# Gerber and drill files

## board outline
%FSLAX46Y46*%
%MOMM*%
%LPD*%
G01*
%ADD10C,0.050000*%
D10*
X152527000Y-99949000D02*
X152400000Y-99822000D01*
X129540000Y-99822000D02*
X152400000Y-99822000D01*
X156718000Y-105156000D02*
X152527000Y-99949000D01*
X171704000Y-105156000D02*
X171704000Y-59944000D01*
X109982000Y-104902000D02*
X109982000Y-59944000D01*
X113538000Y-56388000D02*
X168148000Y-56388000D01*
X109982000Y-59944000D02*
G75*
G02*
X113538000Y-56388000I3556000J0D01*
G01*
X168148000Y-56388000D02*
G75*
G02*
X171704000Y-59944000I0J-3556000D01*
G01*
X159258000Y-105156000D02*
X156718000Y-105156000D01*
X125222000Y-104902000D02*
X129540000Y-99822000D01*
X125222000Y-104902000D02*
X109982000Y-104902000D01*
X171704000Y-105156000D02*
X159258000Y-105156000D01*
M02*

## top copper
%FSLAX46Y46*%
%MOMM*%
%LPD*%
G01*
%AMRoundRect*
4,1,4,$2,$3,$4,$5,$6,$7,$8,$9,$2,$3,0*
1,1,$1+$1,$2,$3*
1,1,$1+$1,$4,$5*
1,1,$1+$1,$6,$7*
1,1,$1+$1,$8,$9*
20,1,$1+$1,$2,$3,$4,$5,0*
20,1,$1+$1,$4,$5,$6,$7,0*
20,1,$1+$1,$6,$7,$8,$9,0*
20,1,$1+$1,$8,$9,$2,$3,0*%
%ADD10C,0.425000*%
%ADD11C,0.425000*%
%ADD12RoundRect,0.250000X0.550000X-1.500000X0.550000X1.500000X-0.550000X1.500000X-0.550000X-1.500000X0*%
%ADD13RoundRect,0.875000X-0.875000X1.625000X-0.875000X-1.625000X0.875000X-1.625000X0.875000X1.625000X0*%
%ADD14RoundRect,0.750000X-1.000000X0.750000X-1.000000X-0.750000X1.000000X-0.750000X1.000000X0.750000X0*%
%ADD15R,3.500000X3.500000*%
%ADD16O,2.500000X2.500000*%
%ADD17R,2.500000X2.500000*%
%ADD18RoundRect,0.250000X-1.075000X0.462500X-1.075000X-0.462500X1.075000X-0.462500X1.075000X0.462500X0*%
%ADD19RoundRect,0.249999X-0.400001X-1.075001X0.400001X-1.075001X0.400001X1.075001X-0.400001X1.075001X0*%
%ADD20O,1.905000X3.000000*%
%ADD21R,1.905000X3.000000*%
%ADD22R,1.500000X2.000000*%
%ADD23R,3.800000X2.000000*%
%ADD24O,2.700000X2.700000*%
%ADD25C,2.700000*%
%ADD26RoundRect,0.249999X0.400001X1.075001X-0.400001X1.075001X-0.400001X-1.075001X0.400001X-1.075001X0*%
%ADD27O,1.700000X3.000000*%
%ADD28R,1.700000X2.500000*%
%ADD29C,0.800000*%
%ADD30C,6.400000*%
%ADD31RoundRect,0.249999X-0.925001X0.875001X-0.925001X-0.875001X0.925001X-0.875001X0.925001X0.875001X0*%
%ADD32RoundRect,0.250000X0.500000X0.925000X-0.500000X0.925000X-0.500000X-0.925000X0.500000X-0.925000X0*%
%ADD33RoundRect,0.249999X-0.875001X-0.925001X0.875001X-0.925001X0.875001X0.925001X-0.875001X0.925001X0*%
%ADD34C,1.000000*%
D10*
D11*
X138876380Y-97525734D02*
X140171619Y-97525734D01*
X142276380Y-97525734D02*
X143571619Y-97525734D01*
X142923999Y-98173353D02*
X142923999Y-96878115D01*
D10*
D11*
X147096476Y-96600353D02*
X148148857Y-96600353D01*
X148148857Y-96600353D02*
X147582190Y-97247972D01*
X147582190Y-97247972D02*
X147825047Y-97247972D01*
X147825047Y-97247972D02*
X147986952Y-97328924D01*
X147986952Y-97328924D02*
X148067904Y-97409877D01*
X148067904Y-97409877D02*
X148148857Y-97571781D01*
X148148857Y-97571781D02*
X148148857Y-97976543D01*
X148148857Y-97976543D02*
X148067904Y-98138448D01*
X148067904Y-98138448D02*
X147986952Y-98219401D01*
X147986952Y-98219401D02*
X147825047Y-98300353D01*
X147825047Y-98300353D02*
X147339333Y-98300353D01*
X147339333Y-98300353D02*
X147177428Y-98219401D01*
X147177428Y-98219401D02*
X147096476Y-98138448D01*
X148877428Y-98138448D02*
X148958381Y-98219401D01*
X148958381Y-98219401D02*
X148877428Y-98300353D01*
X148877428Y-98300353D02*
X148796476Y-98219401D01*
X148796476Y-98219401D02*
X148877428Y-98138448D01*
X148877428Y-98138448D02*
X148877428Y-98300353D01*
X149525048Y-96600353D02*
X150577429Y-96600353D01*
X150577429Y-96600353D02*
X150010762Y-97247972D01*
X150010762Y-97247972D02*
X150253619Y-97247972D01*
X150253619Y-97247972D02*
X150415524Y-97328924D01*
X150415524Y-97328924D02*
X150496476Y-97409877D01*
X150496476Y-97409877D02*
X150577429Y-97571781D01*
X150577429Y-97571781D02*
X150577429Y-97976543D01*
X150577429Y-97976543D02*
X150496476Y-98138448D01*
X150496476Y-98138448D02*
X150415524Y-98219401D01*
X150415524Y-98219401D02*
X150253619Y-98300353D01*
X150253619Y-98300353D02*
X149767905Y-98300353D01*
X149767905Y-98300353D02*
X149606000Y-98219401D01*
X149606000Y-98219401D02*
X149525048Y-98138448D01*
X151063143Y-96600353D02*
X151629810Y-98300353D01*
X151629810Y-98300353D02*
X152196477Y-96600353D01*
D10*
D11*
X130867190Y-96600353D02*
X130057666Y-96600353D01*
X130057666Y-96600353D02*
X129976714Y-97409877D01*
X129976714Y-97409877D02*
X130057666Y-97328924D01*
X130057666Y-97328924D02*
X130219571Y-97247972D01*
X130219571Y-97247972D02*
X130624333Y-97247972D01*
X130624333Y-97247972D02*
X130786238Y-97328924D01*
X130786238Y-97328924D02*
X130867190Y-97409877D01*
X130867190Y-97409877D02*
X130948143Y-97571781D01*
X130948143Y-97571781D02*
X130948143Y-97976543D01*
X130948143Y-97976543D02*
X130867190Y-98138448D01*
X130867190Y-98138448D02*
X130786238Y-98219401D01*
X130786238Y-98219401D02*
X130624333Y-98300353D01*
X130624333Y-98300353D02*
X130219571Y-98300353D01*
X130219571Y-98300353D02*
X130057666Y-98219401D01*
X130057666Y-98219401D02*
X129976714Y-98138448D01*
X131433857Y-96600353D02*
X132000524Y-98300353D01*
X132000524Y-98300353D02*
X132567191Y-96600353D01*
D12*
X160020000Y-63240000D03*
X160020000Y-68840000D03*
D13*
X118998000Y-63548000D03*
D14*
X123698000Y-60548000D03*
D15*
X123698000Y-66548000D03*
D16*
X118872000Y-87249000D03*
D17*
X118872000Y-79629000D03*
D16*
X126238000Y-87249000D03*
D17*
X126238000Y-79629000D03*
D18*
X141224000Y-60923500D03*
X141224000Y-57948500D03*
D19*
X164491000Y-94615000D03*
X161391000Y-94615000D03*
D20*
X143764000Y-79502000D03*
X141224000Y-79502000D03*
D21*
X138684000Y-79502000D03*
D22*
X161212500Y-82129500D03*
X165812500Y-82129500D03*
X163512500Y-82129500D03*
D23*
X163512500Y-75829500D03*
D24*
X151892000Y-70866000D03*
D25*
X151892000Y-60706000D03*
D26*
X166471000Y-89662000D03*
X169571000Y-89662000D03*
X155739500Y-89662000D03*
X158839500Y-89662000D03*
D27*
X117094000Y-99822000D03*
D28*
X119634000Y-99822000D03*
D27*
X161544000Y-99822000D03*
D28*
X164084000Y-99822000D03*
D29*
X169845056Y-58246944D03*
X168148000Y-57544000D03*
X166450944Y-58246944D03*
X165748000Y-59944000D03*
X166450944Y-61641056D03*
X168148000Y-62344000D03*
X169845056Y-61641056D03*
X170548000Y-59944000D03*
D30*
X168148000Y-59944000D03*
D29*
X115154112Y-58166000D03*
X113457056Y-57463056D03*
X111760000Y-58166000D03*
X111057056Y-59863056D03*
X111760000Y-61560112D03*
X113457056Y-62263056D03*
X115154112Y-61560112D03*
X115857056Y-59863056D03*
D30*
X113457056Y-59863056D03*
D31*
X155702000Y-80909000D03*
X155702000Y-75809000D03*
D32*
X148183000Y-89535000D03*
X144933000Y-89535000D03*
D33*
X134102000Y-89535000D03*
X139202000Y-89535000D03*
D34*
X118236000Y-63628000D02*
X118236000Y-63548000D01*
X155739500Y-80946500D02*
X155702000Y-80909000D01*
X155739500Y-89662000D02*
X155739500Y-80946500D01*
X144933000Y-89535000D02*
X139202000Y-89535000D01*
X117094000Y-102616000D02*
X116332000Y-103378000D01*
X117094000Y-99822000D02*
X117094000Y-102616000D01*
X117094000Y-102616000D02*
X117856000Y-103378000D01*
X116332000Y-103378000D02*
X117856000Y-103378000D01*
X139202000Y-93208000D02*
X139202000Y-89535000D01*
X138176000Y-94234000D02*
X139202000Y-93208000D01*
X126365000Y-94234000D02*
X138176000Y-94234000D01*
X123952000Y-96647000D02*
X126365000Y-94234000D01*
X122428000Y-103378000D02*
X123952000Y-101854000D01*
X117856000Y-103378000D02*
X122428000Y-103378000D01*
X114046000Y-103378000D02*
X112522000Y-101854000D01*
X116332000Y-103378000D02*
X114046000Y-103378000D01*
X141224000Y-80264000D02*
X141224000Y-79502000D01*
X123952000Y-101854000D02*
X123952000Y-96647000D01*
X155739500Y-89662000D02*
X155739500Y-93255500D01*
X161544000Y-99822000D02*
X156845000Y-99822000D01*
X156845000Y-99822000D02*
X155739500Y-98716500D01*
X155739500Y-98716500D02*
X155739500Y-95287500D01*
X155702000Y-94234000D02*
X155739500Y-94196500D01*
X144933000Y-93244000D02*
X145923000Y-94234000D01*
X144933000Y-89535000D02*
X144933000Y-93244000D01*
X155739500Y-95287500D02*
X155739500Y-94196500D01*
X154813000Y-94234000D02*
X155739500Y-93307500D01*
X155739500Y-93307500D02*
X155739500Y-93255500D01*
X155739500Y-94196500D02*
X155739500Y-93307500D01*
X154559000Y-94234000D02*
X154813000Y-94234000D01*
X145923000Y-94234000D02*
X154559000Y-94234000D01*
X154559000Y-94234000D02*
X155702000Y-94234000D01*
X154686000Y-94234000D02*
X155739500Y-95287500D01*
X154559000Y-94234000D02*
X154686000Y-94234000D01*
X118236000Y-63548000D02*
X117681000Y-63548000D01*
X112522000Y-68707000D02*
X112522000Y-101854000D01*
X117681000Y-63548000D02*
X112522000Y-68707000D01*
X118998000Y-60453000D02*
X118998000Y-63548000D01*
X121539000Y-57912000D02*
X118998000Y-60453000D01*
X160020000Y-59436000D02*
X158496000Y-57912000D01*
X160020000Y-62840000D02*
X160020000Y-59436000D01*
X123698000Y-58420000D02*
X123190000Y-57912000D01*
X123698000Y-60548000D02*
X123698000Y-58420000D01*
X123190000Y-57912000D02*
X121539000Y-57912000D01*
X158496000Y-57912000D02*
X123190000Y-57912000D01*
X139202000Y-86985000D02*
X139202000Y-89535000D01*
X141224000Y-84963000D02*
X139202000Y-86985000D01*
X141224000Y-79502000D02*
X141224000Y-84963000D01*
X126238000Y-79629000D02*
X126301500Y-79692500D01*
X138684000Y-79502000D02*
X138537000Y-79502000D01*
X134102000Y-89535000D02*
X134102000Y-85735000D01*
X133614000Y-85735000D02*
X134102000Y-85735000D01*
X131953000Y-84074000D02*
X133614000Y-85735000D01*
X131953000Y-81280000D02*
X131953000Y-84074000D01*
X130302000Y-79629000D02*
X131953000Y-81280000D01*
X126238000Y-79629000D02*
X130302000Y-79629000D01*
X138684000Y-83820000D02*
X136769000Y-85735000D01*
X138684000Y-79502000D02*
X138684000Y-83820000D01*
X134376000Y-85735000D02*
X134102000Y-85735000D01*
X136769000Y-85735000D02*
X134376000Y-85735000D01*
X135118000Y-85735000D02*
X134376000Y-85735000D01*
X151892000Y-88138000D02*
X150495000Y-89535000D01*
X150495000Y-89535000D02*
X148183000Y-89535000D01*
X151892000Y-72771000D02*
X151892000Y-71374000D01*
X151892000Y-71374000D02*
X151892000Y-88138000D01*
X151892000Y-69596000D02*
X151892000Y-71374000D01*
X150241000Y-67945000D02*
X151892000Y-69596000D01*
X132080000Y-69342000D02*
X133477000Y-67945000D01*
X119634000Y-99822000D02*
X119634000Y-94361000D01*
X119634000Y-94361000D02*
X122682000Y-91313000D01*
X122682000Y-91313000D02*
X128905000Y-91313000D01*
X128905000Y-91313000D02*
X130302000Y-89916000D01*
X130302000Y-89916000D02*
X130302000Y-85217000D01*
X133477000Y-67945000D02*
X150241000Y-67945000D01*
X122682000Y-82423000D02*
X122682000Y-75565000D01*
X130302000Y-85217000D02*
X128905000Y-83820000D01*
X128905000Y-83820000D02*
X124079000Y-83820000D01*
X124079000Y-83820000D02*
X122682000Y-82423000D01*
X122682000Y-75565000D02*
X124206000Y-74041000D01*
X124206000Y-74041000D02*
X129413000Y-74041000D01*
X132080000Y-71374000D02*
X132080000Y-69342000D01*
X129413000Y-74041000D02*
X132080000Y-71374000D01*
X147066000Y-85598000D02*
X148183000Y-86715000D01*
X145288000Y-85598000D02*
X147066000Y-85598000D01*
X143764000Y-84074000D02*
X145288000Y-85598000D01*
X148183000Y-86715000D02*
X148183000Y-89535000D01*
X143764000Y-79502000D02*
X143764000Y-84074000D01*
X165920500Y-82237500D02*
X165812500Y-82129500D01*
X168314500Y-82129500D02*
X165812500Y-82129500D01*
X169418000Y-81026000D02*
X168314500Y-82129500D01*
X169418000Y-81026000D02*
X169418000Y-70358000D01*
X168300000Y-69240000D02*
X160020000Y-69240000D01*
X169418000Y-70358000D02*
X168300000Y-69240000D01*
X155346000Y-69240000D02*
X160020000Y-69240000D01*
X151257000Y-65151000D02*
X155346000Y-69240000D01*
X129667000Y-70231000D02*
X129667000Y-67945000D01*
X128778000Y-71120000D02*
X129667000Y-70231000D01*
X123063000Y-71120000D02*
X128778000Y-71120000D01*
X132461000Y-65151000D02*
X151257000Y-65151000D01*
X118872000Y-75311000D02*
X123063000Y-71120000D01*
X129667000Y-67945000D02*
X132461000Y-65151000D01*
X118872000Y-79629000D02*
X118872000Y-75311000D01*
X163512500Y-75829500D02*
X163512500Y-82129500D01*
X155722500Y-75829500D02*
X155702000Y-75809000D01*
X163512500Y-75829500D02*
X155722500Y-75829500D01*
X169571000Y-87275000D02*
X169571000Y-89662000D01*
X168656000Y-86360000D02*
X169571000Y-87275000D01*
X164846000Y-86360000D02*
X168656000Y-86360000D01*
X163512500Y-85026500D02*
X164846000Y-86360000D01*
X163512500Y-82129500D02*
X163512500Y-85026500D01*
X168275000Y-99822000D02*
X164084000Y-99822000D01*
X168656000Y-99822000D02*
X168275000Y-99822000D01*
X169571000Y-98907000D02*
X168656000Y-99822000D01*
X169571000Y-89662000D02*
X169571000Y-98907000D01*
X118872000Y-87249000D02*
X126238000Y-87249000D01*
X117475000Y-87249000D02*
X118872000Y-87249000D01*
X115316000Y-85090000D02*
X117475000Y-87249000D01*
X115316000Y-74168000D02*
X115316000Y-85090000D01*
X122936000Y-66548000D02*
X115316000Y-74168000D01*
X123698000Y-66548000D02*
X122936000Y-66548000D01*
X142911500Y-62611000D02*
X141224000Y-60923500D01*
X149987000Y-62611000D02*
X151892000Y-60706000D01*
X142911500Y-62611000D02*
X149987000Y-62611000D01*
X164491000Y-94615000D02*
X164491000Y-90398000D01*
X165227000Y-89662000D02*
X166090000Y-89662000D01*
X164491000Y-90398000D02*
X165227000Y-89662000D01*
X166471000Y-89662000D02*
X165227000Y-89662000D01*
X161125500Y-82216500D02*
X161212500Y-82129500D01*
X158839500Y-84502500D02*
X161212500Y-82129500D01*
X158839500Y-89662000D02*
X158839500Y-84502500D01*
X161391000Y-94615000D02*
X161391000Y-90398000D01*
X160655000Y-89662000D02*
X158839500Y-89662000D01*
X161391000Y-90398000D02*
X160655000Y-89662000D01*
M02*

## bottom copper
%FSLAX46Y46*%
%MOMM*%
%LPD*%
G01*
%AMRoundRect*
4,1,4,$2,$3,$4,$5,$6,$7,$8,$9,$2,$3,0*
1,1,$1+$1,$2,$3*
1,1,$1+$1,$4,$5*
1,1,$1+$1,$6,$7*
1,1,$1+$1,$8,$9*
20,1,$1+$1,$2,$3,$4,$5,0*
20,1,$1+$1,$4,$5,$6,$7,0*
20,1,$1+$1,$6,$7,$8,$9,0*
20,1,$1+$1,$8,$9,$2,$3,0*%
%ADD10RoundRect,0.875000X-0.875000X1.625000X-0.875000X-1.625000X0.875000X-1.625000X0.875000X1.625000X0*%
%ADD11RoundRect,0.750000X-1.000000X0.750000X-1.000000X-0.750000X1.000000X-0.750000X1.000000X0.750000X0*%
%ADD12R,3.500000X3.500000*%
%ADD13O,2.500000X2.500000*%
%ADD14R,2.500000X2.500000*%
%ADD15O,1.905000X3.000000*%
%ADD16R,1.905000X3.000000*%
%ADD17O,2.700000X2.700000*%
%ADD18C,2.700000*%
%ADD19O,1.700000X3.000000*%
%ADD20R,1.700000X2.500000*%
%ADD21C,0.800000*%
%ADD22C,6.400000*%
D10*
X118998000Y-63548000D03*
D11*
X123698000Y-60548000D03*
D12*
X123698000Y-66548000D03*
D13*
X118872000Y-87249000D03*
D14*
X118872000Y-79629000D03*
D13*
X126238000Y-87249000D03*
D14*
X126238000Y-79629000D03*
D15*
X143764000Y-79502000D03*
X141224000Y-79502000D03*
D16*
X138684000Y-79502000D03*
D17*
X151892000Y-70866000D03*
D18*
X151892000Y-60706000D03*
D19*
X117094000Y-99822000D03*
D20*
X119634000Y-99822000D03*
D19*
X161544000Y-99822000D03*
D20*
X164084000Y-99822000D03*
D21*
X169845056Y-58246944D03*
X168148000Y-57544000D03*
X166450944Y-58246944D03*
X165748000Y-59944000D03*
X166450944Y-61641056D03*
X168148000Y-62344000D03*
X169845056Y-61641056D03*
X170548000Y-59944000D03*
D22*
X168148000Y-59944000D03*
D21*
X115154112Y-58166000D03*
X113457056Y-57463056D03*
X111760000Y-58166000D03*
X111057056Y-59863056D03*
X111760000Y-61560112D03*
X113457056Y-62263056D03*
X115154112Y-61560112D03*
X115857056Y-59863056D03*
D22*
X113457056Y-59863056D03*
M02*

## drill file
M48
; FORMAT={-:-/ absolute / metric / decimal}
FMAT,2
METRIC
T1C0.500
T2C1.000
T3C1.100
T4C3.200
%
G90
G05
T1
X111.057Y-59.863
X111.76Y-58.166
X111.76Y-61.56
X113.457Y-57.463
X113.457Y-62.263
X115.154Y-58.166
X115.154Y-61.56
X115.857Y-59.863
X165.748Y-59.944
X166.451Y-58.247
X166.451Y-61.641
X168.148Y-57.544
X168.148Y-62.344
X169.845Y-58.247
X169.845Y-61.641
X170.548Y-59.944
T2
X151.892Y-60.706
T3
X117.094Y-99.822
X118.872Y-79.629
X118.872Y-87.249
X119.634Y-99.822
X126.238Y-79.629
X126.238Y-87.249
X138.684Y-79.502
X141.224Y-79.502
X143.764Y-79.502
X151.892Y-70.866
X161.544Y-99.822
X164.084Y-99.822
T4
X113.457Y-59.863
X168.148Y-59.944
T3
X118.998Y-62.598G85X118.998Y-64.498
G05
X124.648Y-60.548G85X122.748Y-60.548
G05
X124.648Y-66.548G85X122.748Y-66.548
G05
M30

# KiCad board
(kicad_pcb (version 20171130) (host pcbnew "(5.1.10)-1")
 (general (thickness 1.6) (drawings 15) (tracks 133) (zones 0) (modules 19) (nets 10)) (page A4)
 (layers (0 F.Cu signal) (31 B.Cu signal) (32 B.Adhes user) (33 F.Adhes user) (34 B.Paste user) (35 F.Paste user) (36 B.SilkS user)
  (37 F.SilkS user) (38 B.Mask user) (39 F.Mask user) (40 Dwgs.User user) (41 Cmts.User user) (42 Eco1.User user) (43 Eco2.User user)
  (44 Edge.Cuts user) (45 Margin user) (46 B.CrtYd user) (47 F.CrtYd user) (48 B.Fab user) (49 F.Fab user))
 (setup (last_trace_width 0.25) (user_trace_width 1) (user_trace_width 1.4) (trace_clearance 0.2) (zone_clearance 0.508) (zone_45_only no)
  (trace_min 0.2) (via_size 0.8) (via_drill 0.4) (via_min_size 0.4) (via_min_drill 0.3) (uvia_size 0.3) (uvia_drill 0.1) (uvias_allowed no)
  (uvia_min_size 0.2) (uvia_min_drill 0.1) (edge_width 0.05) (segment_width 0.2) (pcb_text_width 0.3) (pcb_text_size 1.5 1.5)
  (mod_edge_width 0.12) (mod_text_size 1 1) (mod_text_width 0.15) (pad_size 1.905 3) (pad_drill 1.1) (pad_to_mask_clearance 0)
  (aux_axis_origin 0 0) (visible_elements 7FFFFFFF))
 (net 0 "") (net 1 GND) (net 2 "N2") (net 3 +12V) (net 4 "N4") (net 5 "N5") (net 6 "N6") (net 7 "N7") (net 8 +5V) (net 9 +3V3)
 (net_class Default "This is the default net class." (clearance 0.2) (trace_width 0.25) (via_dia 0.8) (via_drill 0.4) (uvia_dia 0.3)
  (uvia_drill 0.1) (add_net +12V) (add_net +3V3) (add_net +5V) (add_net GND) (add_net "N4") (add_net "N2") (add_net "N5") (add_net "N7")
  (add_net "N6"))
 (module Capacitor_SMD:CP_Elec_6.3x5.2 (layer F.Cu) (at 160.02 66.04 90)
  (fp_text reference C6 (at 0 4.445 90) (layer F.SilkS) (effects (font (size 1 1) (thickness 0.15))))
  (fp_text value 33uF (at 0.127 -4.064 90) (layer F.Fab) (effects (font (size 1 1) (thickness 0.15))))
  (pad 2 smd roundrect (at 2.8 0 90) (size 3.5 1.6) (layers F.Cu F.Paste F.Mask) (roundrect_rratio 0.15625) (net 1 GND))
  (pad 1 smd roundrect (at -2.8 0 90) (size 3.5 1.6) (layers F.Cu F.Paste F.Mask) (roundrect_rratio 0.15625) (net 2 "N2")))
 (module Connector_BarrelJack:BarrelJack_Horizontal (layer F.Cu) (at 123.698 66.548 270)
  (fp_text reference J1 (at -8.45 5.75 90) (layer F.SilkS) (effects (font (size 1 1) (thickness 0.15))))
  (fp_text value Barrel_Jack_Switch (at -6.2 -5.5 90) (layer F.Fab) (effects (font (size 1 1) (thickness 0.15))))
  (pad 3 thru_hole roundrect (at -3 4.7 270) (size 5 3.5) (drill oval 3 1.1) (layers *.Cu *.Mask) (roundrect_rratio 0.25) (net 1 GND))
  (pad 2 thru_hole roundrect (at -6 0 270) (size 3 3.5) (drill oval 1.1 3) (layers *.Cu *.Mask) (roundrect_rratio 0.25) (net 1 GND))
  (pad 1 thru_hole rect (at 0 0 270) (size 3.5 3.5) (drill oval 1.1 3) (layers *.Cu *.Mask) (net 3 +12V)))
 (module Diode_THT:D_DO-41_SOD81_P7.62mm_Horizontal (layer F.Cu) (at 118.872 79.629 270)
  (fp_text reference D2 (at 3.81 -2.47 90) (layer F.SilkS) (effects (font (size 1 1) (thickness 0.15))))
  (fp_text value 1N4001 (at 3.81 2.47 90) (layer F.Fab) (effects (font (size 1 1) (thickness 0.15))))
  (pad 2 thru_hole oval (at 7.62 0 270) (size 2.5 2.5) (drill 1.1) (layers *.Cu *.Mask) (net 3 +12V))
  (pad 1 thru_hole rect (at 0 0 270) (size 2.5 2.5) (drill 1.1) (layers *.Cu *.Mask) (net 2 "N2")))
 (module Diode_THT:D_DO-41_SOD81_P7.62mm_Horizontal (layer F.Cu) (at 126.238 79.629 270)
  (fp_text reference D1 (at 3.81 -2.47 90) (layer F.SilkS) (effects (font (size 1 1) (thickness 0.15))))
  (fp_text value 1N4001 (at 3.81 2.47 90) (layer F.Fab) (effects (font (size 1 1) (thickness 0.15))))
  (pad 2 thru_hole oval (at 7.62 0 270) (size 2.5 2.5) (drill 1.1) (layers *.Cu *.Mask) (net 3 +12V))
  (pad 1 thru_hole rect (at 0 0 270) (size 2.5 2.5) (drill 1.1) (layers *.Cu *.Mask) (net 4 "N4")))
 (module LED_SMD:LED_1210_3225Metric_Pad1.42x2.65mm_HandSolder (layer F.Cu) (at 141.224 59.436 270)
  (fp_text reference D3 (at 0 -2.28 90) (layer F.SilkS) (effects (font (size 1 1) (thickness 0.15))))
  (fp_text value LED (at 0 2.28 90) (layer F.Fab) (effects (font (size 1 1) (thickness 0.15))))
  (pad 2 smd roundrect (at 1.4875 0 270) (size 1.425 2.65) (layers F.Cu F.Paste F.Mask) (roundrect_rratio 0.1754385964912281) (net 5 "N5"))
  (pad 1 smd roundrect (at -1.4875 0 270) (size 1.425 2.65) (layers F.Cu F.Paste F.Mask) (roundrect_rratio 0.1754385964912281) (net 1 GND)))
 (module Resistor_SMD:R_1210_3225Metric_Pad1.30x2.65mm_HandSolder (layer F.Cu) (at 162.941 94.615)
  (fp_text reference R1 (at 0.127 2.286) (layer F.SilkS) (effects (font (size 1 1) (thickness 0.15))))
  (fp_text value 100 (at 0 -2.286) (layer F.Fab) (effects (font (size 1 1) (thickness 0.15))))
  (pad 2 smd roundrect (at 1.55 0) (size 1.3 2.65) (layers F.Cu F.Paste F.Mask) (roundrect_rratio 0.1923069230769231) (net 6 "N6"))
  (pad 1 smd roundrect (at -1.55 0) (size 1.3 2.65) (layers F.Cu F.Paste F.Mask) (roundrect_rratio 0.1923069230769231) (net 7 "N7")))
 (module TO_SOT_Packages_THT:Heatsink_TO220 (layer F.Cu) (at 141.224 75.438)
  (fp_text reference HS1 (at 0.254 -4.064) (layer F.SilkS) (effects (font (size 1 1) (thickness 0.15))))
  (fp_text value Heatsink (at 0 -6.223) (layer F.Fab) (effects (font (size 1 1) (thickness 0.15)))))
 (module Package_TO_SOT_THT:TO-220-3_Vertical (layer F.Cu) (at 138.684 79.502)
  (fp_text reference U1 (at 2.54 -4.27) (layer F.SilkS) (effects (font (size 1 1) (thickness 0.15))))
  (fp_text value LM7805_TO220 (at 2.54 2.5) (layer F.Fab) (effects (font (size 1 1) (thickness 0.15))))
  (pad 3 thru_hole oval (at 5.08 0) (size 1.905 3) (drill 1.1) (layers *.Cu *.Mask) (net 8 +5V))
  (pad 2 thru_hole oval (at 2.54 0) (size 1.905 3) (drill 1.1) (layers *.Cu *.Mask) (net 1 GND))
  (pad 1 thru_hole rect (at 0 0) (size 1.905 3) (drill 1.1) (layers *.Cu *.Mask) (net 4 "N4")))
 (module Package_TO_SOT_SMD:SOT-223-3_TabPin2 (layer F.Cu) (at 163.5125 78.9795 90)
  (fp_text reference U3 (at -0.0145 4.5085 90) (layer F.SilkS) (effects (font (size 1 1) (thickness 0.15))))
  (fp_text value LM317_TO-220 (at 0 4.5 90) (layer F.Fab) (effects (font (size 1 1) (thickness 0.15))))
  (pad 1 smd rect (at -3.15 -2.3 90) (size 2 1.5) (layers F.Cu F.Paste F.Mask) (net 7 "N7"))
  (pad 3 smd rect (at -3.15 2.3 90) (size 2 1.5) (layers F.Cu F.Paste F.Mask) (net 2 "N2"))
  (pad 2 smd rect (at -3.15 0 90) (size 2 1.5) (layers F.Cu F.Paste F.Mask) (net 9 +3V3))
  (pad 2 smd rect (at 3.15 0 90) (size 2 3.8) (layers F.Cu F.Paste F.Mask) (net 9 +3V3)))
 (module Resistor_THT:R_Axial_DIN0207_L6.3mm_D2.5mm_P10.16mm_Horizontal (layer F.Cu) (at 151.892 60.706 270)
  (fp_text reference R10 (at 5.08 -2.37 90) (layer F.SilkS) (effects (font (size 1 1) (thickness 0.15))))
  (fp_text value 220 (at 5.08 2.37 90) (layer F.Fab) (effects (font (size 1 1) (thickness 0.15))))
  (pad 2 thru_hole oval (at 10.16 0 270) (size 2.7 2.7) (drill 1.1) (layers *.Cu *.Mask) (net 8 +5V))
  (pad 1 thru_hole circle (at 0 0 270) (size 2.7 2.7) (drill 1) (layers *.Cu *.Mask) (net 5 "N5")))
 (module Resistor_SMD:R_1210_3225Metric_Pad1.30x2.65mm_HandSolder (layer F.Cu) (at 168.021 89.662 180)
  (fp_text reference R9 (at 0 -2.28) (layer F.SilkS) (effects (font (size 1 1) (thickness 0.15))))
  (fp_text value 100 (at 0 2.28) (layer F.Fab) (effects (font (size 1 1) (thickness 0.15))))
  (pad 2 smd roundrect (at 1.55 0 180) (size 1.3 2.65) (layers F.Cu F.Paste F.Mask) (roundrect_rratio 0.1923069230769231) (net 6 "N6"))
  (pad 1 smd roundrect (at -1.55 0 180) (size 1.3 2.65) (layers F.Cu F.Paste F.Mask) (roundrect_rratio 0.1923069230769231) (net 9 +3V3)))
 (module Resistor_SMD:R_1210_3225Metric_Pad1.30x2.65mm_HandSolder (layer F.Cu) (at 157.2895 89.662 180)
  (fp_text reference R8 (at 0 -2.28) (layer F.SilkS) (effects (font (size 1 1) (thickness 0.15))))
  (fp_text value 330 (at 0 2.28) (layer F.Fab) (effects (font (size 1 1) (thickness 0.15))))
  (pad 2 smd roundrect (at 1.55 0 180) (size 1.3 2.65) (layers F.Cu F.Paste F.Mask) (roundrect_rratio 0.1923069230769231) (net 1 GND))
  (pad 1 smd roundrect (at -1.55 0 180) (size 1.3 2.65) (layers F.Cu F.Paste F.Mask) (roundrect_rratio 0.1923069230769231) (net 7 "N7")))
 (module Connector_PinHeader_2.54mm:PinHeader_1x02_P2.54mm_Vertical (layer B.Cu) (at 119.634 99.822 90)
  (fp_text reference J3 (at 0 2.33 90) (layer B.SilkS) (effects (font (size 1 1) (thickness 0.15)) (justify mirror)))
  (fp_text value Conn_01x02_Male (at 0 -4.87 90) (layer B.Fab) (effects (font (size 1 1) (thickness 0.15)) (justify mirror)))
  (pad 2 thru_hole oval (at 0 -2.54 90) (size 3 1.7) (drill 1.1) (layers *.Cu *.Mask) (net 1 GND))
  (pad 1 thru_hole rect (at 0 0 90) (size 2.5 1.7) (drill 1.1) (layers *.Cu *.Mask) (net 8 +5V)))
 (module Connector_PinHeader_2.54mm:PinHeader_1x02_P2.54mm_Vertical (layer B.Cu) (at 164.084 99.822 90)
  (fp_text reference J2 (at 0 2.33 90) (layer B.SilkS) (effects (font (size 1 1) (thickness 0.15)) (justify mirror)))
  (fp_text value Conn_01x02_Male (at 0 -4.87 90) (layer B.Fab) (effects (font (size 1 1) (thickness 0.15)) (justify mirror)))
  (pad 2 thru_hole oval (at 0 -2.54 90) (size 3 1.7) (drill 1.1) (layers *.Cu *.Mask) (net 1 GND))
  (pad 1 thru_hole rect (at 0 0 90) (size 2.5 1.7) (drill 1.1) (layers *.Cu *.Mask) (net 9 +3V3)))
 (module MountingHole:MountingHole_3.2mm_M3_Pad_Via (layer F.Cu) (at 168.148 59.944)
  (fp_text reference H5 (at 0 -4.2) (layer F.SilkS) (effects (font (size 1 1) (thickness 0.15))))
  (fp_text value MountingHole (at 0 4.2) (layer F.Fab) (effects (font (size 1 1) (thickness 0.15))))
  (pad 1 thru_hole circle (at 1.697056 -1.697056) (size 0.8 0.8) (drill 0.5) (layers *.Cu *.Mask))
  (pad 1 thru_hole circle (at 0 -2.4) (size 0.8 0.8) (drill 0.5) (layers *.Cu *.Mask))
  (pad 1 thru_hole circle (at -1.697056 -1.697056) (size 0.8 0.8) (drill 0.5) (layers *.Cu *.Mask))
  (pad 1 thru_hole circle (at -2.4 0) (size 0.8 0.8) (drill 0.5) (layers *.Cu *.Mask))
  (pad 1 thru_hole circle (at -1.697056 1.697056) (size 0.8 0.8) (drill 0.5) (layers *.Cu *.Mask))
  (pad 1 thru_hole circle (at 0 2.4) (size 0.8 0.8) (drill 0.5) (layers *.Cu *.Mask))
  (pad 1 thru_hole circle (at 1.697056 1.697056) (size 0.8 0.8) (drill 0.5) (layers *.Cu *.Mask))
  (pad 1 thru_hole circle (at 2.4 0) (size 0.8 0.8) (drill 0.5) (layers *.Cu *.Mask))
  (pad 1 thru_hole circle (at 0 0) (size 6.4 6.4) (drill 3.2) (layers *.Cu *.Mask)))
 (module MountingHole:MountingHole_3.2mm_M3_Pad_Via (layer F.Cu) (at 113.457056 59.863056)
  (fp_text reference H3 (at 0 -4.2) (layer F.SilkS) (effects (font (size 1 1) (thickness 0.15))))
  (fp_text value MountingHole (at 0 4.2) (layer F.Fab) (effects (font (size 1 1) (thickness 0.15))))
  (pad 1 thru_hole circle (at 1.697056 -1.697056) (size 0.8 0.8) (drill 0.5) (layers *.Cu *.Mask))
  (pad 1 thru_hole circle (at 0 -2.4) (size 0.8 0.8) (drill 0.5) (layers *.Cu *.Mask))
  (pad 1 thru_hole circle (at -1.697056 -1.697056) (size 0.8 0.8) (drill 0.5) (layers *.Cu *.Mask))
  (pad 1 thru_hole circle (at -2.4 0) (size 0.8 0.8) (drill 0.5) (layers *.Cu *.Mask))
  (pad 1 thru_hole circle (at -1.697056 1.697056) (size 0.8 0.8) (drill 0.5) (layers *.Cu *.Mask))
  (pad 1 thru_hole circle (at 0 2.4) (size 0.8 0.8) (drill 0.5) (layers *.Cu *.Mask))
  (pad 1 thru_hole circle (at 1.697056 1.697056) (size 0.8 0.8) (drill 0.5) (layers *.Cu *.Mask))
  (pad 1 thru_hole circle (at 2.4 0) (size 0.8 0.8) (drill 0.5) (layers *.Cu *.Mask))
  (pad 1 thru_hole circle (at 0 0) (size 6.4 6.4) (drill 3.2) (layers *.Cu *.Mask)))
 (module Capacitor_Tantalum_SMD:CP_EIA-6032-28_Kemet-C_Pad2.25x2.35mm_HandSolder (layer F.Cu) (at 155.702 78.359 270)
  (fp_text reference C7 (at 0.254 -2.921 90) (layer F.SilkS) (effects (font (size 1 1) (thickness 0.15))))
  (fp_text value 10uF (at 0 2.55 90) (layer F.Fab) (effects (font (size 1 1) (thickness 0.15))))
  (pad 2 smd roundrect (at 2.55 0 270) (size 2.25 2.35) (layers F.Cu F.Paste F.Mask) (roundrect_rratio 0.1111106666666667) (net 1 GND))
  (pad 1 smd roundrect (at -2.55 0 270) (size 2.25 2.35) (layers F.Cu F.Paste F.Mask) (roundrect_rratio 0.1111106666666667) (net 9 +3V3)))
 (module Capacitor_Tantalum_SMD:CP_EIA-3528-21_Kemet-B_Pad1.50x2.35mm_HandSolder (layer F.Cu) (at 146.558 89.535 180)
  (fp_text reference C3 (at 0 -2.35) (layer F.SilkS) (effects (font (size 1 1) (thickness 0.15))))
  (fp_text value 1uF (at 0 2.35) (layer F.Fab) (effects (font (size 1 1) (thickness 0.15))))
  (pad 1 smd roundrect (at -1.625 0 180) (size 1.5 2.35) (layers F.Cu F.Paste F.Mask) (roundrect_rratio 0.1666666666666667) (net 8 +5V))
  (pad 2 smd roundrect (at 1.625 0 180) (size 1.5 2.35) (layers F.Cu F.Paste F.Mask) (roundrect_rratio 0.1666666666666667) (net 1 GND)))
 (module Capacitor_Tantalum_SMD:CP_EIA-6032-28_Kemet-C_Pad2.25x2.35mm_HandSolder (layer F.Cu) (at 136.652 89.535)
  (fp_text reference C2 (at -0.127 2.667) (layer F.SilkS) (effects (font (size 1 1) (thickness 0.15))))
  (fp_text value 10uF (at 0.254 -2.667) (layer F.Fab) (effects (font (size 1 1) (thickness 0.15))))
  (pad 1 smd roundrect (at -2.55 0) (size 2.25 2.35) (layers F.Cu F.Paste F.Mask) (roundrect_rratio 0.1111106666666667) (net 4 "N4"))
  (pad 2 smd roundrect (at 2.55 0) (size 2.25 2.35) (layers F.Cu F.Paste F.Mask) (roundrect_rratio 0.1111106666666667) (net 1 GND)))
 (gr_line (start 152.527 99.949) (end 152.4 99.822) (layer Edge.Cuts) (width 0.05))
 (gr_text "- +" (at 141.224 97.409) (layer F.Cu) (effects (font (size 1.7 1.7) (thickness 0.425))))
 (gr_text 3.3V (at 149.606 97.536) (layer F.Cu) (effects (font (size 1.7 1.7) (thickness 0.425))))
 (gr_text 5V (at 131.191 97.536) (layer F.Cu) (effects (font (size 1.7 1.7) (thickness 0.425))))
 (gr_line (start 129.54 99.822) (end 152.4 99.822) (layer Edge.Cuts) (width 0.05))
 (gr_line (start 156.718 105.156) (end 152.527 99.949) (layer Edge.Cuts) (width 0.05))
 (gr_line (start 171.704 105.156) (end 171.704 59.944) (layer Edge.Cuts) (width 0.05))
 (gr_line (start 109.982 104.902) (end 109.982 59.944) (layer Edge.Cuts) (width 0.05))
 (gr_line (start 113.538 56.388) (end 168.148 56.388) (layer Edge.Cuts) (width 0.05))
 (gr_arc (start 113.538 59.944) (end 113.538 56.388) (angle -90) (layer Edge.Cuts) (width 0.05))
 (gr_arc (start 168.148 59.944) (end 171.704 59.944) (angle -90) (layer Edge.Cuts) (width 0.05))
 (gr_line (start 159.258 105.156) (end 156.718 105.156) (layer Edge.Cuts) (width 0.05))
 (gr_line (start 125.222 104.902) (end 129.54 99.822) (layer Edge.Cuts) (width 0.05))
 (gr_line (start 125.222 104.902) (end 109.982 104.902) (layer Edge.Cuts) (width 0.05))
 (gr_line (start 171.704 105.156) (end 159.258 105.156) (layer Edge.Cuts) (width 0.05))
 (segment (start 118.236 63.628) (end 118.236 63.548) (width 1) (layer F.Cu) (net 1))
 (segment (start 155.7395 80.9465) (end 155.702 80.909) (width 1) (layer F.Cu) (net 1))
 (segment (start 155.7395 89.662) (end 155.7395 80.9465) (width 1) (layer F.Cu) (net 1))
 (segment (start 144.933 89.535) (end 139.202 89.535) (width 1) (layer F.Cu) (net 1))
 (segment (start 117.094 102.616) (end 116.332 103.378) (width 1) (layer F.Cu) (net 1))
 (segment (start 117.094 99.822) (end 117.094 102.616) (width 1) (layer F.Cu) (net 1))
 (segment (start 117.094 102.616) (end 117.856 103.378) (width 1) (layer F.Cu) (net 1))
 (segment (start 116.332 103.378) (end 117.856 103.378) (width 1) (layer F.Cu) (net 1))
 (segment (start 139.202 93.208) (end 139.202 89.535) (width 1) (layer F.Cu) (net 1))
 (segment (start 138.176 94.234) (end 139.202 93.208) (width 1) (layer F.Cu) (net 1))
 (segment (start 126.365 94.234) (end 138.176 94.234) (width 1) (layer F.Cu) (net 1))
 (segment (start 123.952 96.647) (end 126.365 94.234) (width 1) (layer F.Cu) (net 1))
 (segment (start 122.428 103.378) (end 123.952 101.854) (width 1) (layer F.Cu) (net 1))
 (segment (start 117.856 103.378) (end 122.428 103.378) (width 1) (layer F.Cu) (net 1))
 (segment (start 114.046 103.378) (end 112.522 101.854) (width 1) (layer F.Cu) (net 1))
 (segment (start 116.332 103.378) (end 114.046 103.378) (width 1) (layer F.Cu) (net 1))
 (segment (start 141.224 80.264) (end 141.224 79.502) (width 1) (layer F.Cu) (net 1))
 (segment (start 123.952 101.854) (end 123.952 96.647) (width 1) (layer F.Cu) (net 1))
 (segment (start 155.7395 89.662) (end 155.7395 93.2555) (width 1) (layer F.Cu) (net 1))
 (segment (start 161.544 99.822) (end 156.845 99.822) (width 1) (layer F.Cu) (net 1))
 (segment (start 156.845 99.822) (end 155.7395 98.7165) (width 1) (layer F.Cu) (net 1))
 (segment (start 155.7395 98.7165) (end 155.7395 95.2875) (width 1) (layer F.Cu) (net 1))
 (segment (start 155.702 94.234) (end 155.7395 94.1965) (width 1) (layer F.Cu) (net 1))
 (segment (start 144.933 93.244) (end 145.923 94.234) (width 1) (layer F.Cu) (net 1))
 (segment (start 144.933 89.535) (end 144.933 93.244) (width 1) (layer F.Cu) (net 1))
 (segment (start 155.7395 95.2875) (end 155.7395 94.1965) (width 1) (layer F.Cu) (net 1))
 (segment (start 154.813 94.234) (end 155.7395 93.3075) (width 1) (layer F.Cu) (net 1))
 (segment (start 155.7395 93.3075) (end 155.7395 93.2555) (width 1) (layer F.Cu) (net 1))
 (segment (start 155.7395 94.1965) (end 155.7395 93.3075) (width 1) (layer F.Cu) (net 1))
 (segment (start 154.559 94.234) (end 154.813 94.234) (width 1) (layer F.Cu) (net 1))
 (segment (start 145.923 94.234) (end 154.559 94.234) (width 1) (layer F.Cu) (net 1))
 (segment (start 154.559 94.234) (end 155.702 94.234) (width 1) (layer F.Cu) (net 1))
 (segment (start 154.686 94.234) (end 155.7395 95.2875) (width 1) (layer F.Cu) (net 1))
 (segment (start 154.559 94.234) (end 154.686 94.234) (width 1) (layer F.Cu) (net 1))
 (segment (start 118.236 63.548) (end 117.681 63.548) (width 1) (layer F.Cu) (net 1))
 (segment (start 112.522 68.707) (end 112.522 101.854) (width 1) (layer F.Cu) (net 1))
 (segment (start 117.681 63.548) (end 112.522 68.707) (width 1) (layer F.Cu) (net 1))
 (segment (start 118.998 60.453) (end 118.998 63.548) (width 1) (layer F.Cu) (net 1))
 (segment (start 121.539 57.912) (end 118.998 60.453) (width 1) (layer F.Cu) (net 1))
 (segment (start 160.02 59.436) (end 158.496 57.912) (width 1) (layer F.Cu) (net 1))
 (segment (start 160.02 62.84) (end 160.02 59.436) (width 1) (layer F.Cu) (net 1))
 (segment (start 123.698 58.42) (end 123.19 57.912) (width 1) (layer F.Cu) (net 1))
 (segment (start 123.698 60.548) (end 123.698 58.42) (width 1) (layer F.Cu) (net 1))
 (segment (start 123.19 57.912) (end 121.539 57.912) (width 1) (layer F.Cu) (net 1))
 (segment (start 158.496 57.912) (end 123.19 57.912) (width 1) (layer F.Cu) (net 1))
 (segment (start 139.202 86.985) (end 139.202 89.535) (width 1) (layer F.Cu) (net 1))
 (segment (start 141.224 84.963) (end 139.202 86.985) (width 1) (layer F.Cu) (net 1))
 (segment (start 141.224 79.502) (end 141.224 84.963) (width 1) (layer F.Cu) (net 1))
 (segment (start 126.238 79.629) (end 126.3015 79.6925) (width 1) (layer F.Cu) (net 4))
 (segment (start 138.684 79.502) (end 138.537 79.502) (width 1) (layer F.Cu) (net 4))
 (segment (start 134.102 89.535) (end 134.102 85.735) (width 1) (layer F.Cu) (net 4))
 (segment (start 133.614 85.735) (end 134.102 85.735) (width 1) (layer F.Cu) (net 4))
 (segment (start 131.953 84.074) (end 133.614 85.735) (width 1) (layer F.Cu) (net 4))
 (segment (start 131.953 81.28) (end 131.953 84.074) (width 1) (layer F.Cu) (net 4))
 (segment (start 130.302 79.629) (end 131.953 81.28) (width 1) (layer F.Cu) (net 4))
 (segment (start 126.238 79.629) (end 130.302 79.629) (width 1) (layer F.Cu) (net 4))
 (segment (start 138.684 83.82) (end 136.769 85.735) (width 1) (layer F.Cu) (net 4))
 (segment (start 138.684 79.502) (end 138.684 83.82) (width 1) (layer F.Cu) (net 4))
 (segment (start 134.376 85.735) (end 134.102 85.735) (width 1) (layer F.Cu) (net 4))
 (segment (start 136.769 85.735) (end 134.376 85.735) (width 1) (layer F.Cu) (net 4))
 (segment (start 135.118 85.735) (end 134.376 85.735) (width 1) (layer F.Cu) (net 4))
 (segment (start 151.892 88.138) (end 150.495 89.535) (width 1) (layer F.Cu) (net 8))
 (segment (start 150.495 89.535) (end 148.183 89.535) (width 1) (layer F.Cu) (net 8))
 (segment (start 151.892 72.771) (end 151.892 71.374) (width 1) (layer F.Cu) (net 8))
 (segment (start 151.892 71.374) (end 151.892 88.138) (width 1) (layer F.Cu) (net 8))
 (segment (start 151.892 69.596) (end 151.892 71.374) (width 1) (layer F.Cu) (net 8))
 (segment (start 150.241 67.945) (end 151.892 69.596) (width 1) (layer F.Cu) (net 8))
 (segment (start 132.08 69.342) (end 133.477 67.945) (width 1) (layer F.Cu) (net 8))
 (segment (start 119.634 99.822) (end 119.634 94.361) (width 1) (layer F.Cu) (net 8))
 (segment (start 119.634 94.361) (end 122.682 91.313) (width 1) (layer F.Cu) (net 8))
 (segment (start 122.682 91.313) (end 128.905 91.313) (width 1) (layer F.Cu) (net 8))
 (segment (start 128.905 91.313) (end 130.302 89.916) (width 1) (layer F.Cu) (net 8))
 (segment (start 130.302 89.916) (end 130.302 85.217) (width 1) (layer F.Cu) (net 8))
 (segment (start 133.477 67.945) (end 150.241 67.945) (width 1) (layer F.Cu) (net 8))
 (segment (start 122.682 82.423) (end 122.682 75.565) (width 1) (layer F.Cu) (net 8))
 (segment (start 130.302 85.217) (end 128.905 83.82) (width 1) (layer F.Cu) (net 8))
 (segment (start 128.905 83.82) (end 124.079 83.82) (width 1) (layer F.Cu) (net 8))
 (segment (start 124.079 83.82) (end 122.682 82.423) (width 1) (layer F.Cu) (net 8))
 (segment (start 122.682 75.565) (end 124.206 74.041) (width 1) (layer F.Cu) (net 8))
 (segment (start 124.206 74.041) (end 129.413 74.041) (width 1) (layer F.Cu) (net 8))
 (segment (start 132.08 71.374) (end 132.08 69.342) (width 1) (layer F.Cu) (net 8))
 (segment (start 129.413 74.041) (end 132.08 71.374) (width 1) (layer F.Cu) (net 8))
 (segment (start 147.066 85.598) (end 148.183 86.715) (width 1) (layer F.Cu) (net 8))
 (segment (start 145.288 85.598) (end 147.066 85.598) (width 1) (layer F.Cu) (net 8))
 (segment (start 143.764 84.074) (end 145.288 85.598) (width 1) (layer F.Cu) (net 8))
 (segment (start 148.183 86.715) (end 148.183 89.535) (width 1) (layer F.Cu) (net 8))
 (segment (start 143.764 79.502) (end 143.764 84.074) (width 1) (layer F.Cu) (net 8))
 (segment (start 165.9205 82.2375) (end 165.8125 82.1295) (width 1) (layer F.Cu) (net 2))
 (segment (start 168.3145 82.1295) (end 165.8125 82.1295) (width 1) (layer F.Cu) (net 2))
 (segment (start 169.418 81.026) (end 168.3145 82.1295) (width 1) (layer F.Cu) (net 2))
 (segment (start 169.418 81.026) (end 169.418 70.358) (width 1) (layer F.Cu) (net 2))
 (segment (start 168.3 69.24) (end 160.02 69.24) (width 1) (layer F.Cu) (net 2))
 (segment (start 169.418 70.358) (end 168.3 69.24) (width 1) (layer F.Cu) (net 2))
 (segment (start 155.346 69.24) (end 160.02 69.24) (width 1) (layer F.Cu) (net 2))
 (segment (start 151.257 65.151) (end 155.346 69.24) (width 1) (layer F.Cu) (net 2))
 (segment (start 129.667 70.231) (end 129.667 67.945) (width 1) (layer F.Cu) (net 2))
 (segment (start 128.778 71.12) (end 129.667 70.231) (width 1) (layer F.Cu) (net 2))
 (segment (start 123.063 71.12) (end 128.778 71.12) (width 1) (layer F.Cu) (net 2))
 (segment (start 132.461 65.151) (end 151.257 65.151) (width 1) (layer F.Cu) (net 2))
 (segment (start 118.872 75.311) (end 123.063 71.12) (width 1) (layer F.Cu) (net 2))
 (segment (start 129.667 67.945) (end 132.461 65.151) (width 1) (layer F.Cu) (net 2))
 (segment (start 118.872 79.629) (end 118.872 75.311) (width 1) (layer F.Cu) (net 2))
 (segment (start 163.5125 75.8295) (end 163.5125 82.1295) (width 1) (layer F.Cu) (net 9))
 (segment (start 155.7225 75.8295) (end 155.702 75.809) (width 1) (layer F.Cu) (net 9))
 (segment (start 163.5125 75.8295) (end 155.7225 75.8295) (width 1) (layer F.Cu) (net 9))
 (segment (start 169.571 87.275) (end 169.571 89.662) (width 1) (layer F.Cu) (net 9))
 (segment (start 168.656 86.36) (end 169.571 87.275) (width 1) (layer F.Cu) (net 9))
 (segment (start 164.846 86.36) (end 168.656 86.36) (width 1) (layer F.Cu) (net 9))
 (segment (start 163.5125 85.0265) (end 164.846 86.36) (width 1) (layer F.Cu) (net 9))
 (segment (start 163.5125 82.1295) (end 163.5125 85.0265) (width 1) (layer F.Cu) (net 9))
 (segment (start 168.275 99.822) (end 164.084 99.822) (width 1) (layer F.Cu) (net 9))
 (segment (start 168.656 99.822) (end 168.275 99.822) (width 1) (layer F.Cu) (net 9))
 (segment (start 169.571 98.907) (end 168.656 99.822) (width 1) (layer F.Cu) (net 9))
 (segment (start 169.571 89.662) (end 169.571 98.907) (width 1) (layer F.Cu) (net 9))
 (segment (start 118.872 87.249) (end 126.238 87.249) (width 1) (layer F.Cu) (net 3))
 (segment (start 117.475 87.249) (end 118.872 87.249) (width 1) (layer F.Cu) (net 3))
 (segment (start 115.316 85.09) (end 117.475 87.249) (width 1) (layer F.Cu) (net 3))
 (segment (start 115.316 74.168) (end 115.316 85.09) (width 1) (layer F.Cu) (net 3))
 (segment (start 122.936 66.548) (end 115.316 74.168) (width 1) (layer F.Cu) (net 3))
 (segment (start 123.698 66.548) (end 122.936 66.548) (width 1) (layer F.Cu) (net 3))
 (segment (start 142.9115 62.611) (end 141.224 60.9235) (width 1) (layer F.Cu) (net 5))
 (segment (start 149.987 62.611) (end 151.892 60.706) (width 1) (layer F.Cu) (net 5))
 (segment (start 142.9115 62.611) (end 149.987 62.611) (width 1) (layer F.Cu) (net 5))
 (segment (start 164.491 94.615) (end 164.491 90.398) (width 1) (layer F.Cu) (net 6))
 (segment (start 165.227 89.662) (end 166.09 89.662) (width 1) (layer F.Cu) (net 6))
 (segment (start 164.491 90.398) (end 165.227 89.662) (width 1) (layer F.Cu) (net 6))
 (segment (start 166.471 89.662) (end 165.227 89.662) (width 1) (layer F.Cu) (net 6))
 (segment (start 161.1255 82.2165) (end 161.2125 82.1295) (width 1) (layer F.Cu) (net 7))
 (segment (start 158.8395 84.5025) (end 161.2125 82.1295) (width 1) (layer F.Cu) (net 7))
 (segment (start 158.8395 89.662) (end 158.8395 84.5025) (width 1) (layer F.Cu) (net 7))
 (segment (start 161.391 94.615) (end 161.391 90.398) (width 1) (layer F.Cu) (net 7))
 (segment (start 160.655 89.662) (end 158.8395 89.662) (width 1) (layer F.Cu) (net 7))
 (segment (start 161.391 90.398) (end 160.655 89.662) (width 1) (layer F.Cu) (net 7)))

